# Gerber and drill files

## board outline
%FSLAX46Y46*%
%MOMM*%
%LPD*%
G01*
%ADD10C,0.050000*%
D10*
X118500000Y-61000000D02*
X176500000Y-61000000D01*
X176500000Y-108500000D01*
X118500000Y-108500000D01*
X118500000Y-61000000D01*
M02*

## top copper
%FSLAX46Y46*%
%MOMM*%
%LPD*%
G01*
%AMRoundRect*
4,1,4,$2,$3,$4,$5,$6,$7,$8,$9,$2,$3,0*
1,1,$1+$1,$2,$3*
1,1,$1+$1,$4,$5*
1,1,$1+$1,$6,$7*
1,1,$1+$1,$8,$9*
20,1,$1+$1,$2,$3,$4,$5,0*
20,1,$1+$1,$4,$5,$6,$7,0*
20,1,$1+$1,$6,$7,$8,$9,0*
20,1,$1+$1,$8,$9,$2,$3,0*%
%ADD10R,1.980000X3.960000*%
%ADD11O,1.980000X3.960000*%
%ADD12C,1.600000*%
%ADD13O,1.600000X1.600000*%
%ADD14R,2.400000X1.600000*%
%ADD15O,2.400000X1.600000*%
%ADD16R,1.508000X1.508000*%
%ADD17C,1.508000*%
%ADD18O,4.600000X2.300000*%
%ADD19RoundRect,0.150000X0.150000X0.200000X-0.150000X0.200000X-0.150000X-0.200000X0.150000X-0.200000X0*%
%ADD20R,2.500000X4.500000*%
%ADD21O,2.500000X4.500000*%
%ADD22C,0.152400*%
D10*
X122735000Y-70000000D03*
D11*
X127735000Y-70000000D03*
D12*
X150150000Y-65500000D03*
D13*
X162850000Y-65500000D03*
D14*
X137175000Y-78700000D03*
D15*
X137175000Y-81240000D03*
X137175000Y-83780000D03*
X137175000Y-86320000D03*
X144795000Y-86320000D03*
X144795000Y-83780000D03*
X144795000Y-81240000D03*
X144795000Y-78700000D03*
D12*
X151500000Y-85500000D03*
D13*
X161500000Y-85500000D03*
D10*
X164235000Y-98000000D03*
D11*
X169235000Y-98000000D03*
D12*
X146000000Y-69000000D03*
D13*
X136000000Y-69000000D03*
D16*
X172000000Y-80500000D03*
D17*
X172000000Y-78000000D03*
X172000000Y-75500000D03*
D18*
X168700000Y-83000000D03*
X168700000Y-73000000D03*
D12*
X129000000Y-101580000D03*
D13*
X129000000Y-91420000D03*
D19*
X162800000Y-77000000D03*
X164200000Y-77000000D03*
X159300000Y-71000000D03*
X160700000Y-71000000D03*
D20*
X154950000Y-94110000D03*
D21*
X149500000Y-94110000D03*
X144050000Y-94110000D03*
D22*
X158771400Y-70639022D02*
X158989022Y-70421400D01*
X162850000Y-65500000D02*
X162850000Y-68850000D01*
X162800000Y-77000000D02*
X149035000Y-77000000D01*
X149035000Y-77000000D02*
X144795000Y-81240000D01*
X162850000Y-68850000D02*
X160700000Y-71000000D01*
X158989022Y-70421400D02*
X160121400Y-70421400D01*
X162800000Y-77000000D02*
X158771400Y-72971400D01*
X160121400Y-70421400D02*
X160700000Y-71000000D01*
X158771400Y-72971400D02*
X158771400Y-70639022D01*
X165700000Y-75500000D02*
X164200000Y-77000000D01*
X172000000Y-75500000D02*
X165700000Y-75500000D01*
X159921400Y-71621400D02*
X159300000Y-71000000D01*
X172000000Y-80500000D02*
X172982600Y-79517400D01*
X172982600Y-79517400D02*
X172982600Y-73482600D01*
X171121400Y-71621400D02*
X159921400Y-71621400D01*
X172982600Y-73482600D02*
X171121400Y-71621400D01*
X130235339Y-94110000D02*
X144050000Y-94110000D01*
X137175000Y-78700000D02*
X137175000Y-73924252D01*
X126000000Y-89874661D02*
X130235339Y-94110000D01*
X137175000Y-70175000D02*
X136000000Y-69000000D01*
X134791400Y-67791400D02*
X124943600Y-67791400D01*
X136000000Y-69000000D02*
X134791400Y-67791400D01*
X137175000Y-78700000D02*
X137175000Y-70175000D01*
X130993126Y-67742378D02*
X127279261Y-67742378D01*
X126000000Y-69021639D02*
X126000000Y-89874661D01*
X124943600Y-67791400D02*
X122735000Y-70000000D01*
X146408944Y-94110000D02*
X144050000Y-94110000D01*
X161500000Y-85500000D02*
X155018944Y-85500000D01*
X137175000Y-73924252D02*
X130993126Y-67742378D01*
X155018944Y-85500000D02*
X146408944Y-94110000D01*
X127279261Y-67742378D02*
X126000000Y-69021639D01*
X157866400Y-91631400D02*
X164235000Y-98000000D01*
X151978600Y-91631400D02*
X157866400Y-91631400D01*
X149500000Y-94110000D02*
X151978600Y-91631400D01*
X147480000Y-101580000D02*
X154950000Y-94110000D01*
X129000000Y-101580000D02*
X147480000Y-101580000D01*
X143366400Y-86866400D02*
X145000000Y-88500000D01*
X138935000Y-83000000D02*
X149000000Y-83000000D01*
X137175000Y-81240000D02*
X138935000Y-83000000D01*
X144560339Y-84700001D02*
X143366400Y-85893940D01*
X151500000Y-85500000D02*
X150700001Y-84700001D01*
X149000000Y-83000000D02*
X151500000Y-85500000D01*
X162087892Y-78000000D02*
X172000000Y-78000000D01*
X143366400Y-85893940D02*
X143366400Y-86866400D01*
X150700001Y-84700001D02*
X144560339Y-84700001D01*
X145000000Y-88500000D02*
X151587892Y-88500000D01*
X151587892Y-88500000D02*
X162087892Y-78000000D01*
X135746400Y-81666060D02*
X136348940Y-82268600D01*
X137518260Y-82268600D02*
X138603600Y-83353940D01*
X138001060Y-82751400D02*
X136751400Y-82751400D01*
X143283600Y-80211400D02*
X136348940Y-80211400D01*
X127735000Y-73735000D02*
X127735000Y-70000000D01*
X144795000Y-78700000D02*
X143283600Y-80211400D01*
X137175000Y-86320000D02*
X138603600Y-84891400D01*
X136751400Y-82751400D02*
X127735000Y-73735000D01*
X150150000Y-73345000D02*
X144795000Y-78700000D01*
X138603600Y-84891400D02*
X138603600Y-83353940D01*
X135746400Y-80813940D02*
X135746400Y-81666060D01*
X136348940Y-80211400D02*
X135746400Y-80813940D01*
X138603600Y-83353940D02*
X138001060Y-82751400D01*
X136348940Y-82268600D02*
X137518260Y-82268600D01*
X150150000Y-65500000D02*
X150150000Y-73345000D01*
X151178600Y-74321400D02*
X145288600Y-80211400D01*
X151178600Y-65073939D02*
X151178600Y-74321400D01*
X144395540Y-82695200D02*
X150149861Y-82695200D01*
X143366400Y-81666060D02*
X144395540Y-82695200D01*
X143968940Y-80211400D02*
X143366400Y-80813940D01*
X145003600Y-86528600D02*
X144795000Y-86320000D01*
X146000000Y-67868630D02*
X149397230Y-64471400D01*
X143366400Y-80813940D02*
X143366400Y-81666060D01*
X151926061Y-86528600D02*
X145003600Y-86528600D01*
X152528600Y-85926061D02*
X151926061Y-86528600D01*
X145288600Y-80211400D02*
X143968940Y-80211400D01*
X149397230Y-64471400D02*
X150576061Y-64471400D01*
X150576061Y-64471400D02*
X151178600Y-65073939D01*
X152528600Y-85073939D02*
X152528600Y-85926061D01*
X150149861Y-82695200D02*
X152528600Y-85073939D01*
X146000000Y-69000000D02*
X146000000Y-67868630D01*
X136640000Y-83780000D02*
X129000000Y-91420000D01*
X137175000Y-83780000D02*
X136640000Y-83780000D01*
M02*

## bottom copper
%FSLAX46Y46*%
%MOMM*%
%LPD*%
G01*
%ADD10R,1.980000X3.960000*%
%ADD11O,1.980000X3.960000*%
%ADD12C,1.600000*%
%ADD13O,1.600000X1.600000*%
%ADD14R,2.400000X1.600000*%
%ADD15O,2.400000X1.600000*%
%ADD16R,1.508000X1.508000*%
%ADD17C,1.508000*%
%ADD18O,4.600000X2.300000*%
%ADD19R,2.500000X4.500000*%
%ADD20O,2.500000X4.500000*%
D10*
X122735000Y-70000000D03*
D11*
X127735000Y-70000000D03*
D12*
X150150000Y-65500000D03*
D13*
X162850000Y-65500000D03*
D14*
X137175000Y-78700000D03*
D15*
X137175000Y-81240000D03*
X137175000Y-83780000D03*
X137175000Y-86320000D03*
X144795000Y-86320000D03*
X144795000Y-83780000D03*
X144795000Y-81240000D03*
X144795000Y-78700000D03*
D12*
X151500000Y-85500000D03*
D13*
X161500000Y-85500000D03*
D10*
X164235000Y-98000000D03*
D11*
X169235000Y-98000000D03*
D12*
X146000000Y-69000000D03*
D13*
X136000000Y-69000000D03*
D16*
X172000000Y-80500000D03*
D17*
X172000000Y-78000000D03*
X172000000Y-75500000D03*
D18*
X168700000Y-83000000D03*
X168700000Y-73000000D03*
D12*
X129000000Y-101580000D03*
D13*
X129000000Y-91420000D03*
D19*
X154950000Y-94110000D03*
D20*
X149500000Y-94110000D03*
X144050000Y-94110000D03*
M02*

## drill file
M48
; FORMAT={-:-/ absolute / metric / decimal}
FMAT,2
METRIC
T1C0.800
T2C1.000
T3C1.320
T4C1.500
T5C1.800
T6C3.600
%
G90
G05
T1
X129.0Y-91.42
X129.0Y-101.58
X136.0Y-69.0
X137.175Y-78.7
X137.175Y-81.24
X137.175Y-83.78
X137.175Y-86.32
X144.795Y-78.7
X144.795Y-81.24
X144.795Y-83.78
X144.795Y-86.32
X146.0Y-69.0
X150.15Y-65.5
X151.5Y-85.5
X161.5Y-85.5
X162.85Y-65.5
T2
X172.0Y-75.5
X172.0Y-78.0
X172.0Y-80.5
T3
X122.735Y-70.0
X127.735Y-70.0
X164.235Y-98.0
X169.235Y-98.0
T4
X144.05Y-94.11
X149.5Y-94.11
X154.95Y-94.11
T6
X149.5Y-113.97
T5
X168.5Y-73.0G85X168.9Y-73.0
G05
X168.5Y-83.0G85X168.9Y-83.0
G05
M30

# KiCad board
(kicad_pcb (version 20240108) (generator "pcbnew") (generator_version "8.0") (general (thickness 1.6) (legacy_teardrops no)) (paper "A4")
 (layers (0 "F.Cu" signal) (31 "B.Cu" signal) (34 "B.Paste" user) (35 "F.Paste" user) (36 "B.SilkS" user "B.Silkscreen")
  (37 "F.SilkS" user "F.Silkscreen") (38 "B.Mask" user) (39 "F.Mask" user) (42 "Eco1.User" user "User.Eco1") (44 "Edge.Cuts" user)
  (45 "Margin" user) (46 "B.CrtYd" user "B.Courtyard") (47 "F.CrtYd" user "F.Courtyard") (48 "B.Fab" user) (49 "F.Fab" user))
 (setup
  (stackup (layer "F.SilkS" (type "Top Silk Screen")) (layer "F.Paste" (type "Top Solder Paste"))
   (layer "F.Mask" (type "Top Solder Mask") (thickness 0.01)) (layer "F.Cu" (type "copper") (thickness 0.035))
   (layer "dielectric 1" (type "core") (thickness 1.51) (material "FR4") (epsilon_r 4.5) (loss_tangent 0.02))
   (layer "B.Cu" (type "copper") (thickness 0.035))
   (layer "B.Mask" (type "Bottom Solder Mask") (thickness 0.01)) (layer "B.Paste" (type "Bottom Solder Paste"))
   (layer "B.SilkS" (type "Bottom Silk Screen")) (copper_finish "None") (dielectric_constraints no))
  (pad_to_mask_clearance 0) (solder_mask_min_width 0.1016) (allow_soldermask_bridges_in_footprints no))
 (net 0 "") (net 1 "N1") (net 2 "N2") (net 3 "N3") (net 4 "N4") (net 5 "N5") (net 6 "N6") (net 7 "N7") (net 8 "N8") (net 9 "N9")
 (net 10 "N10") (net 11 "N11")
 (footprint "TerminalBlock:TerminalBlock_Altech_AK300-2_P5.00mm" (layer "F.Cu") (at 122.735 70)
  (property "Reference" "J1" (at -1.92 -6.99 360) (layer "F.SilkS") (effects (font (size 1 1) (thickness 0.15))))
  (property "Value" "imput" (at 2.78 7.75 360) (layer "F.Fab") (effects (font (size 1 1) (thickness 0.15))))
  (pad "1" thru_hole rect (at 0 0) (size 1.98 3.96) (drill 1.32) (layers "*.Cu" "*.Mask") (remove_unused_layers no) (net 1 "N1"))
  (pad "2" thru_hole oval (at 5 0) (size 1.98 3.96) (drill 1.32) (layers "*.Cu" "*.Mask") (remove_unused_layers no) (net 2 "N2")))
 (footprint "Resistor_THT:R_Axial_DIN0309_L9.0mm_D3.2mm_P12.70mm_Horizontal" (layer "F.Cu") (at 150.15 65.5)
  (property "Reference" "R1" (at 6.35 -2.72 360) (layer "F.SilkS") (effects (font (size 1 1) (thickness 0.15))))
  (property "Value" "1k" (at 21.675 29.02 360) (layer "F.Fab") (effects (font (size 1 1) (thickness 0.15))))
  (pad "1" thru_hole circle (at 0 0) (size 1.6 1.6) (drill 0.8) (layers "*.Cu" "*.Mask") (remove_unused_layers no) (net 2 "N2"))
  (pad "2" thru_hole oval (at 12.7 0) (size 1.6 1.6) (drill 0.8) (layers "*.Cu" "*.Mask") (remove_unused_layers no) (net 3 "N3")))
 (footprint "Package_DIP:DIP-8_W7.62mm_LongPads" (layer "F.Cu") (at 137.175 78.7)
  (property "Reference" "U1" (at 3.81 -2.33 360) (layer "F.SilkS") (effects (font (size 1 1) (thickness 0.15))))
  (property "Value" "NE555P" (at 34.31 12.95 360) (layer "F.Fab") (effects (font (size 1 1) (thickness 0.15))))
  (pad "1" thru_hole rect (at 0 0) (size 2.4 1.6) (drill 0.8) (layers "*.Cu" "*.Mask") (remove_unused_layers no) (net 1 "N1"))
  (pad "2" thru_hole oval (at 0 2.54) (size 2.4 1.6) (drill 0.8) (layers "*.Cu" "*.Mask") (remove_unused_layers no) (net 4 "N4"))
  (pad "3" thru_hole oval (at 0 5.08) (size 2.4 1.6) (drill 0.8) (layers "*.Cu" "*.Mask") (remove_unused_layers no) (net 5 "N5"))
  (pad "4" thru_hole oval (at 0 7.62) (size 2.4 1.6) (drill 0.8) (layers "*.Cu" "*.Mask") (remove_unused_layers no) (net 2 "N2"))
  (pad "5" thru_hole oval (at 7.62 7.62) (size 2.4 1.6) (drill 0.8) (layers "*.Cu" "*.Mask") (remove_unused_layers no) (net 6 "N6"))
  (pad "6" thru_hole oval (at 7.62 5.08) (size 2.4 1.6) (drill 0.8) (layers "*.Cu" "*.Mask") (remove_unused_layers no) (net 4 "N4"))
  (pad "7" thru_hole oval (at 7.62 2.54) (size 2.4 1.6) (drill 0.8) (layers "*.Cu" "*.Mask") (remove_unused_layers no) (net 3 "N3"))
  (pad "8" thru_hole oval (at 7.62 0) (size 2.4 1.6) (drill 0.8) (layers "*.Cu" "*.Mask") (remove_unused_layers no) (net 2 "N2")))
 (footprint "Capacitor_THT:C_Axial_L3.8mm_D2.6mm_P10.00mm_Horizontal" (layer "F.Cu") (at 151.5 85.5)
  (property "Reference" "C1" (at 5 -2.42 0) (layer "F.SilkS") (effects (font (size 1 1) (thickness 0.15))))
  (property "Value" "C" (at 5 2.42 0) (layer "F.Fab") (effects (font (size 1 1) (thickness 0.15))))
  (pad "1" thru_hole circle (at 0 0) (size 1.6 1.6) (drill 0.8) (layers "*.Cu" "*.Mask") (remove_unused_layers no) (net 4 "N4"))
  (pad "2" thru_hole oval (at 10 0) (size 1.6 1.6) (drill 0.8) (layers "*.Cu" "*.Mask") (remove_unused_layers no) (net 1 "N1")))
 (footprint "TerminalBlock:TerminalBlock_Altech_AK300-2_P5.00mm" (layer "F.Cu") (at 164.235 98)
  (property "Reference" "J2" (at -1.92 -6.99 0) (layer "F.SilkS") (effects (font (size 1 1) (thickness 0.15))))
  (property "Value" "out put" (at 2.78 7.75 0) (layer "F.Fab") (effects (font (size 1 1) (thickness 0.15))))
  (pad "1" thru_hole rect (at 0 0) (size 1.98 3.96) (drill 1.32) (layers "*.Cu" "*.Mask") (remove_unused_layers no) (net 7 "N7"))
  (pad "2" thru_hole oval (at 5 0) (size 1.98 3.96) (drill 1.32) (layers "*.Cu" "*.Mask") (remove_unused_layers no) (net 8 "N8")))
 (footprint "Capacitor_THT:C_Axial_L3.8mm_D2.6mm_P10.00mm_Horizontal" (layer "F.Cu") (at 146 69 180)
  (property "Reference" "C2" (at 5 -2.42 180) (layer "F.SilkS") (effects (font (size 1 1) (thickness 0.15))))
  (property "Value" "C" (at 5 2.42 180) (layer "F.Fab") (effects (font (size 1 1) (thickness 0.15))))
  (pad "1" thru_hole circle (at 0 0 180) (size 1.6 1.6) (drill 0.8) (layers "*.Cu" "*.Mask") (remove_unused_layers no) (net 6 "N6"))
  (pad "2" thru_hole oval (at 10 0 180) (size 1.6 1.6) (drill 0.8) (layers "*.Cu" "*.Mask") (remove_unused_layers no) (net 1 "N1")))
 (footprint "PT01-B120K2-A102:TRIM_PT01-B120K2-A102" (layer "F.Cu") (at 168.7 78 90)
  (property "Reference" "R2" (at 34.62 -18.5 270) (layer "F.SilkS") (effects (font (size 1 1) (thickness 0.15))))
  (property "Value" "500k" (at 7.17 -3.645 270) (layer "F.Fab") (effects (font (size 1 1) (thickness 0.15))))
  (pad "1" thru_hole rect (at -2.5 3.3 90) (size 1.508 1.508) (drill 1) (layers "*.Cu" "*.Mask") (remove_unused_layers no) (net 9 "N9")
   (solder_mask_margin 0.102))
  (pad "2" thru_hole circle (at 0 3.3 90) (size 1.508 1.508) (drill 1) (layers "*.Cu" "*.Mask") (remove_unused_layers no) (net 4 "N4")
   (solder_mask_margin 0.102))
  (pad "3" thru_hole circle (at 2.5 3.3 90) (size 1.508 1.508) (drill 1) (layers "*.Cu" "*.Mask") (remove_unused_layers no) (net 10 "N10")
   (solder_mask_margin 0.102))
  (pad "S1" thru_hole oval (at -5 0 90) (size 2.3 4.6) (drill oval 1.8 2.2) (layers "*.Cu" "*.Mask") (remove_unused_layers no)
   (solder_mask_margin 0.102))
  (pad "S2" thru_hole oval (at 5 0 90) (size 2.3 4.6) (drill oval 1.8 2.2) (layers "*.Cu" "*.Mask") (remove_unused_layers no)
   (solder_mask_margin 0.102)))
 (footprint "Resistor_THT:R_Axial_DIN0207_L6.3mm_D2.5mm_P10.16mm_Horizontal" (layer "F.Cu") (at 129 101.58 90)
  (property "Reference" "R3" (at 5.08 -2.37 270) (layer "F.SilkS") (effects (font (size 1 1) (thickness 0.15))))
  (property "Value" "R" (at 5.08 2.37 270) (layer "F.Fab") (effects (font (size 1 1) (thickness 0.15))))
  (pad "1" thru_hole circle (at 0 0 90) (size 1.6 1.6) (drill 0.8) (layers "*.Cu" "*.Mask") (remove_unused_layers no) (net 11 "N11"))
  (pad "2" thru_hole oval (at 10.16 0 90) (size 1.6 1.6) (drill 0.8) (layers "*.Cu" "*.Mask") (remove_unused_layers no) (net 5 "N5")))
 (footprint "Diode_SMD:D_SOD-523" (layer "F.Cu") (at 163.5 77)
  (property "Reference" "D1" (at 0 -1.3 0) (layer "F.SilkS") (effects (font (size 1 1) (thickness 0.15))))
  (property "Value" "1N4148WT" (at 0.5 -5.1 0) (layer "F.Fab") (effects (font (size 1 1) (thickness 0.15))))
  (pad "1" smd roundrect (at -0.7 0 180) (size 0.6 0.7) (layers "F.Cu" "F.Paste" "F.Mask") (roundrect_rratio 0.25) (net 3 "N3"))
  (pad "2" smd roundrect (at 0.7 0 180) (size 0.6 0.7) (layers "F.Cu" "F.Paste" "F.Mask") (roundrect_rratio 0.25) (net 10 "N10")))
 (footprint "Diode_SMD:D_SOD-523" (layer "F.Cu") (at 160 71)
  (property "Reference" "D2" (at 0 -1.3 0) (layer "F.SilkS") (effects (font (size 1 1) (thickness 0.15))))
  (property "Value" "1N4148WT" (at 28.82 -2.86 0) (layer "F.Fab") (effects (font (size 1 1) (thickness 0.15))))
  (pad "1" smd roundrect (at -0.7 0 180) (size 0.6 0.7) (layers "F.Cu" "F.Paste" "F.Mask") (roundrect_rratio 0.25) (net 9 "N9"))
  (pad "2" smd roundrect (at 0.7 0 180) (size 0.6 0.7) (layers "F.Cu" "F.Paste" "F.Mask") (roundrect_rratio 0.25) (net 3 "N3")))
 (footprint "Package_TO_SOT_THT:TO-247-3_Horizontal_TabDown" (layer "F.Cu") (at 154.95 94.11 180)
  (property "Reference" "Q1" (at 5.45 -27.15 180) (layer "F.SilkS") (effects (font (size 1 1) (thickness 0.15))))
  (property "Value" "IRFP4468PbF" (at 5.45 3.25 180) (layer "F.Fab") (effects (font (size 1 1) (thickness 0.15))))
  (pad "" np_thru_hole oval (at 5.45 -19.86 180) (size 3.6 3.6) (drill 3.6) (layers "*.Cu" "*.Mask"))
  (pad "1" thru_hole rect (at 0 0 180) (size 2.5 4.5) (drill 1.5) (layers "*.Cu" "*.Mask") (remove_unused_layers no) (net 11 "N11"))
  (pad "2" thru_hole oval (at 5.45 0 180) (size 2.5 4.5) (drill 1.5) (layers "*.Cu" "*.Mask") (remove_unused_layers no) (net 7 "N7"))
  (pad "3" thru_hole oval (at 10.9 0 180) (size 2.5 4.5) (drill 1.5) (layers "*.Cu" "*.Mask") (remove_unused_layers no) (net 1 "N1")))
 (gr_rect (start 118.5 61) (end 176.5 108.5) (stroke (width 0.05) (type default)) (fill none) (layer "Edge.Cuts"))
 (segment (start 158.7714 70.639022) (end 158.989022 70.4214) (width 0.1524) (layer "F.Cu") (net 3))
 (segment (start 162.85 65.5) (end 162.85 68.85) (width 0.1524) (layer "F.Cu") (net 3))
 (segment (start 162.8 77) (end 149.035 77) (width 0.1524) (layer "F.Cu") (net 3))
 (segment (start 149.035 77) (end 144.795 81.24) (width 0.1524) (layer "F.Cu") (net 3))
 (segment (start 162.85 68.85) (end 160.7 71) (width 0.1524) (layer "F.Cu") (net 3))
 (segment (start 158.989022 70.4214) (end 160.1214 70.4214) (width 0.1524) (layer "F.Cu") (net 3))
 (segment (start 162.8 77) (end 158.7714 72.9714) (width 0.1524) (layer "F.Cu") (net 3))
 (segment (start 160.1214 70.4214) (end 160.7 71) (width 0.1524) (layer "F.Cu") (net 3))
 (segment (start 158.7714 72.9714) (end 158.7714 70.639022) (width 0.1524) (layer "F.Cu") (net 3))
 (segment (start 165.7 75.5) (end 164.2 77) (width 0.1524) (layer "F.Cu") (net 10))
 (segment (start 172 75.5) (end 165.7 75.5) (width 0.1524) (layer "F.Cu") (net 10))
 (segment (start 159.9214 71.6214) (end 159.3 71) (width 0.1524) (layer "F.Cu") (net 9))
 (segment (start 172 80.5) (end 172.9826 79.5174) (width 0.1524) (layer "F.Cu") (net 9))
 (segment (start 172.9826 79.5174) (end 172.9826 73.4826) (width 0.1524) (layer "F.Cu") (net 9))
 (segment (start 171.1214 71.6214) (end 159.9214 71.6214) (width 0.1524) (layer "F.Cu") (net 9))
 (segment (start 172.9826 73.4826) (end 171.1214 71.6214) (width 0.1524) (layer "F.Cu") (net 9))
 (segment (start 130.235339 94.11) (end 144.05 94.11) (width 0.1524) (layer "F.Cu") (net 1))
 (segment (start 137.175 78.7) (end 137.175 73.924252) (width 0.1524) (layer "F.Cu") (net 1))
 (segment (start 126 89.874661) (end 130.235339 94.11) (width 0.1524) (layer "F.Cu") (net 1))
 (segment (start 137.175 70.175) (end 136 69) (width 0.1524) (layer "F.Cu") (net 1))
 (segment (start 134.7914 67.7914) (end 124.9436 67.7914) (width 0.1524) (layer "F.Cu") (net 1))
 (segment (start 136 69) (end 134.7914 67.7914) (width 0.1524) (layer "F.Cu") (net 1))
 (segment (start 137.175 78.7) (end 137.175 70.175) (width 0.1524) (layer "F.Cu") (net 1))
 (segment (start 130.993126 67.742378) (end 127.279261 67.742378) (width 0.1524) (layer "F.Cu") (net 1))
 (segment (start 126 69.021639) (end 126 89.874661) (width 0.1524) (layer "F.Cu") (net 1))
 (segment (start 124.9436 67.7914) (end 122.735 70) (width 0.1524) (layer "F.Cu") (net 1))
 (segment (start 146.408944 94.11) (end 144.05 94.11) (width 0.1524) (layer "F.Cu") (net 1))
 (segment (start 161.5 85.5) (end 155.018944 85.5) (width 0.1524) (layer "F.Cu") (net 1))
 (segment (start 137.175 73.924252) (end 130.993126 67.742378) (width 0.1524) (layer "F.Cu") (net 1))
 (segment (start 155.018944 85.5) (end 146.408944 94.11) (width 0.1524) (layer "F.Cu") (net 1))
 (segment (start 127.279261 67.742378) (end 126 69.021639) (width 0.1524) (layer "F.Cu") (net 1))
 (segment (start 157.8664 91.6314) (end 164.235 98) (width 0.1524) (layer "F.Cu") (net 7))
 (segment (start 151.9786 91.6314) (end 157.8664 91.6314) (width 0.1524) (layer "F.Cu") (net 7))
 (segment (start 149.5 94.11) (end 151.9786 91.6314) (width 0.1524) (layer "F.Cu") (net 7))
 (segment (start 147.48 101.58) (end 154.95 94.11) (width 0.1524) (layer "F.Cu") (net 11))
 (segment (start 129 101.58) (end 147.48 101.58) (width 0.1524) (layer "F.Cu") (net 11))
 (segment (start 143.3664 86.8664) (end 145 88.5) (width 0.1524) (layer "F.Cu") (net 4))
 (segment (start 138.935 83) (end 149 83) (width 0.1524) (layer "F.Cu") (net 4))
 (segment (start 137.175 81.24) (end 138.935 83) (width 0.1524) (layer "F.Cu") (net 4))
 (segment (start 144.560339 84.700001) (end 143.3664 85.89394) (width 0.1524) (layer "F.Cu") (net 4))
 (segment (start 151.5 85.5) (end 150.700001 84.700001) (width 0.1524) (layer "F.Cu") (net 4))
 (segment (start 149 83) (end 151.5 85.5) (width 0.1524) (layer "F.Cu") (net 4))
 (segment (start 162.087892 78) (end 172 78) (width 0.1524) (layer "F.Cu") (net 4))
 (segment (start 143.3664 85.89394) (end 143.3664 86.8664) (width 0.1524) (layer "F.Cu") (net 4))
 (segment (start 150.700001 84.700001) (end 144.560339 84.700001) (width 0.1524) (layer "F.Cu") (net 4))
 (segment (start 145 88.5) (end 151.587892 88.5) (width 0.1524) (layer "F.Cu") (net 4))
 (segment (start 151.587892 88.5) (end 162.087892 78) (width 0.1524) (layer "F.Cu") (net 4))
 (segment (start 135.7464 81.66606) (end 136.34894 82.2686) (width 0.1524) (layer "F.Cu") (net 2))
 (segment (start 137.51826 82.2686) (end 138.6036 83.35394) (width 0.1524) (layer "F.Cu") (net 2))
 (segment (start 138.00106 82.7514) (end 136.7514 82.7514) (width 0.1524) (layer "F.Cu") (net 2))
 (segment (start 143.2836 80.2114) (end 136.34894 80.2114) (width 0.1524) (layer "F.Cu") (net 2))
 (segment (start 127.735 73.735) (end 127.735 70) (width 0.1524) (layer "F.Cu") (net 2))
 (segment (start 144.795 78.7) (end 143.2836 80.2114) (width 0.1524) (layer "F.Cu") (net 2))
 (segment (start 137.175 86.32) (end 138.6036 84.8914) (width 0.1524) (layer "F.Cu") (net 2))
 (segment (start 136.7514 82.7514) (end 127.735 73.735) (width 0.1524) (layer "F.Cu") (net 2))
 (segment (start 150.15 73.345) (end 144.795 78.7) (width 0.1524) (layer "F.Cu") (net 2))
 (segment (start 138.6036 84.8914) (end 138.6036 83.35394) (width 0.1524) (layer "F.Cu") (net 2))
 (segment (start 135.7464 80.81394) (end 135.7464 81.66606) (width 0.1524) (layer "F.Cu") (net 2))
 (segment (start 136.34894 80.2114) (end 135.7464 80.81394) (width 0.1524) (layer "F.Cu") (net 2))
 (segment (start 138.6036 83.35394) (end 138.00106 82.7514) (width 0.1524) (layer "F.Cu") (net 2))
 (segment (start 136.34894 82.2686) (end 137.51826 82.2686) (width 0.1524) (layer "F.Cu") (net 2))
 (segment (start 150.15 65.5) (end 150.15 73.345) (width 0.1524) (layer "F.Cu") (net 2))
 (segment (start 151.1786 74.3214) (end 145.2886 80.2114) (width 0.1524) (layer "F.Cu") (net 6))
 (segment (start 151.1786 65.073939) (end 151.1786 74.3214) (width 0.1524) (layer "F.Cu") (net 6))
 (segment (start 144.39554 82.6952) (end 150.149861 82.6952) (width 0.1524) (layer "F.Cu") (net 6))
 (segment (start 143.3664 81.66606) (end 144.39554 82.6952) (width 0.1524) (layer "F.Cu") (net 6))
 (segment (start 143.96894 80.2114) (end 143.3664 80.81394) (width 0.1524) (layer "F.Cu") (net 6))
 (segment (start 145.0036 86.5286) (end 144.795 86.32) (width 0.1524) (layer "F.Cu") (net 6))
 (segment (start 146 67.86863) (end 149.39723 64.4714) (width 0.1524) (layer "F.Cu") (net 6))
 (segment (start 143.3664 80.81394) (end 143.3664 81.66606) (width 0.1524) (layer "F.Cu") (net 6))
 (segment (start 151.926061 86.5286) (end 145.0036 86.5286) (width 0.1524) (layer "F.Cu") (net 6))
 (segment (start 152.5286 85.926061) (end 151.926061 86.5286) (width 0.1524) (layer "F.Cu") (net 6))
 (segment (start 145.2886 80.2114) (end 143.96894 80.2114) (width 0.1524) (layer "F.Cu") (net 6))
 (segment (start 149.39723 64.4714) (end 150.576061 64.4714) (width 0.1524) (layer "F.Cu") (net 6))
 (segment (start 150.576061 64.4714) (end 151.1786 65.073939) (width 0.1524) (layer "F.Cu") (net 6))
 (segment (start 152.5286 85.073939) (end 152.5286 85.926061) (width 0.1524) (layer "F.Cu") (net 6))
 (segment (start 150.149861 82.6952) (end 152.5286 85.073939) (width 0.1524) (layer "F.Cu") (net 6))
 (segment (start 146 69) (end 146 67.86863) (width 0.1524) (layer "F.Cu") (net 6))
 (segment (start 136.64 83.78) (end 129 91.42) (width 0.1524) (layer "F.Cu") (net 5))
 (segment (start 137.175 83.78) (end 136.64 83.78) (width 0.1524) (layer "F.Cu") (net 5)))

